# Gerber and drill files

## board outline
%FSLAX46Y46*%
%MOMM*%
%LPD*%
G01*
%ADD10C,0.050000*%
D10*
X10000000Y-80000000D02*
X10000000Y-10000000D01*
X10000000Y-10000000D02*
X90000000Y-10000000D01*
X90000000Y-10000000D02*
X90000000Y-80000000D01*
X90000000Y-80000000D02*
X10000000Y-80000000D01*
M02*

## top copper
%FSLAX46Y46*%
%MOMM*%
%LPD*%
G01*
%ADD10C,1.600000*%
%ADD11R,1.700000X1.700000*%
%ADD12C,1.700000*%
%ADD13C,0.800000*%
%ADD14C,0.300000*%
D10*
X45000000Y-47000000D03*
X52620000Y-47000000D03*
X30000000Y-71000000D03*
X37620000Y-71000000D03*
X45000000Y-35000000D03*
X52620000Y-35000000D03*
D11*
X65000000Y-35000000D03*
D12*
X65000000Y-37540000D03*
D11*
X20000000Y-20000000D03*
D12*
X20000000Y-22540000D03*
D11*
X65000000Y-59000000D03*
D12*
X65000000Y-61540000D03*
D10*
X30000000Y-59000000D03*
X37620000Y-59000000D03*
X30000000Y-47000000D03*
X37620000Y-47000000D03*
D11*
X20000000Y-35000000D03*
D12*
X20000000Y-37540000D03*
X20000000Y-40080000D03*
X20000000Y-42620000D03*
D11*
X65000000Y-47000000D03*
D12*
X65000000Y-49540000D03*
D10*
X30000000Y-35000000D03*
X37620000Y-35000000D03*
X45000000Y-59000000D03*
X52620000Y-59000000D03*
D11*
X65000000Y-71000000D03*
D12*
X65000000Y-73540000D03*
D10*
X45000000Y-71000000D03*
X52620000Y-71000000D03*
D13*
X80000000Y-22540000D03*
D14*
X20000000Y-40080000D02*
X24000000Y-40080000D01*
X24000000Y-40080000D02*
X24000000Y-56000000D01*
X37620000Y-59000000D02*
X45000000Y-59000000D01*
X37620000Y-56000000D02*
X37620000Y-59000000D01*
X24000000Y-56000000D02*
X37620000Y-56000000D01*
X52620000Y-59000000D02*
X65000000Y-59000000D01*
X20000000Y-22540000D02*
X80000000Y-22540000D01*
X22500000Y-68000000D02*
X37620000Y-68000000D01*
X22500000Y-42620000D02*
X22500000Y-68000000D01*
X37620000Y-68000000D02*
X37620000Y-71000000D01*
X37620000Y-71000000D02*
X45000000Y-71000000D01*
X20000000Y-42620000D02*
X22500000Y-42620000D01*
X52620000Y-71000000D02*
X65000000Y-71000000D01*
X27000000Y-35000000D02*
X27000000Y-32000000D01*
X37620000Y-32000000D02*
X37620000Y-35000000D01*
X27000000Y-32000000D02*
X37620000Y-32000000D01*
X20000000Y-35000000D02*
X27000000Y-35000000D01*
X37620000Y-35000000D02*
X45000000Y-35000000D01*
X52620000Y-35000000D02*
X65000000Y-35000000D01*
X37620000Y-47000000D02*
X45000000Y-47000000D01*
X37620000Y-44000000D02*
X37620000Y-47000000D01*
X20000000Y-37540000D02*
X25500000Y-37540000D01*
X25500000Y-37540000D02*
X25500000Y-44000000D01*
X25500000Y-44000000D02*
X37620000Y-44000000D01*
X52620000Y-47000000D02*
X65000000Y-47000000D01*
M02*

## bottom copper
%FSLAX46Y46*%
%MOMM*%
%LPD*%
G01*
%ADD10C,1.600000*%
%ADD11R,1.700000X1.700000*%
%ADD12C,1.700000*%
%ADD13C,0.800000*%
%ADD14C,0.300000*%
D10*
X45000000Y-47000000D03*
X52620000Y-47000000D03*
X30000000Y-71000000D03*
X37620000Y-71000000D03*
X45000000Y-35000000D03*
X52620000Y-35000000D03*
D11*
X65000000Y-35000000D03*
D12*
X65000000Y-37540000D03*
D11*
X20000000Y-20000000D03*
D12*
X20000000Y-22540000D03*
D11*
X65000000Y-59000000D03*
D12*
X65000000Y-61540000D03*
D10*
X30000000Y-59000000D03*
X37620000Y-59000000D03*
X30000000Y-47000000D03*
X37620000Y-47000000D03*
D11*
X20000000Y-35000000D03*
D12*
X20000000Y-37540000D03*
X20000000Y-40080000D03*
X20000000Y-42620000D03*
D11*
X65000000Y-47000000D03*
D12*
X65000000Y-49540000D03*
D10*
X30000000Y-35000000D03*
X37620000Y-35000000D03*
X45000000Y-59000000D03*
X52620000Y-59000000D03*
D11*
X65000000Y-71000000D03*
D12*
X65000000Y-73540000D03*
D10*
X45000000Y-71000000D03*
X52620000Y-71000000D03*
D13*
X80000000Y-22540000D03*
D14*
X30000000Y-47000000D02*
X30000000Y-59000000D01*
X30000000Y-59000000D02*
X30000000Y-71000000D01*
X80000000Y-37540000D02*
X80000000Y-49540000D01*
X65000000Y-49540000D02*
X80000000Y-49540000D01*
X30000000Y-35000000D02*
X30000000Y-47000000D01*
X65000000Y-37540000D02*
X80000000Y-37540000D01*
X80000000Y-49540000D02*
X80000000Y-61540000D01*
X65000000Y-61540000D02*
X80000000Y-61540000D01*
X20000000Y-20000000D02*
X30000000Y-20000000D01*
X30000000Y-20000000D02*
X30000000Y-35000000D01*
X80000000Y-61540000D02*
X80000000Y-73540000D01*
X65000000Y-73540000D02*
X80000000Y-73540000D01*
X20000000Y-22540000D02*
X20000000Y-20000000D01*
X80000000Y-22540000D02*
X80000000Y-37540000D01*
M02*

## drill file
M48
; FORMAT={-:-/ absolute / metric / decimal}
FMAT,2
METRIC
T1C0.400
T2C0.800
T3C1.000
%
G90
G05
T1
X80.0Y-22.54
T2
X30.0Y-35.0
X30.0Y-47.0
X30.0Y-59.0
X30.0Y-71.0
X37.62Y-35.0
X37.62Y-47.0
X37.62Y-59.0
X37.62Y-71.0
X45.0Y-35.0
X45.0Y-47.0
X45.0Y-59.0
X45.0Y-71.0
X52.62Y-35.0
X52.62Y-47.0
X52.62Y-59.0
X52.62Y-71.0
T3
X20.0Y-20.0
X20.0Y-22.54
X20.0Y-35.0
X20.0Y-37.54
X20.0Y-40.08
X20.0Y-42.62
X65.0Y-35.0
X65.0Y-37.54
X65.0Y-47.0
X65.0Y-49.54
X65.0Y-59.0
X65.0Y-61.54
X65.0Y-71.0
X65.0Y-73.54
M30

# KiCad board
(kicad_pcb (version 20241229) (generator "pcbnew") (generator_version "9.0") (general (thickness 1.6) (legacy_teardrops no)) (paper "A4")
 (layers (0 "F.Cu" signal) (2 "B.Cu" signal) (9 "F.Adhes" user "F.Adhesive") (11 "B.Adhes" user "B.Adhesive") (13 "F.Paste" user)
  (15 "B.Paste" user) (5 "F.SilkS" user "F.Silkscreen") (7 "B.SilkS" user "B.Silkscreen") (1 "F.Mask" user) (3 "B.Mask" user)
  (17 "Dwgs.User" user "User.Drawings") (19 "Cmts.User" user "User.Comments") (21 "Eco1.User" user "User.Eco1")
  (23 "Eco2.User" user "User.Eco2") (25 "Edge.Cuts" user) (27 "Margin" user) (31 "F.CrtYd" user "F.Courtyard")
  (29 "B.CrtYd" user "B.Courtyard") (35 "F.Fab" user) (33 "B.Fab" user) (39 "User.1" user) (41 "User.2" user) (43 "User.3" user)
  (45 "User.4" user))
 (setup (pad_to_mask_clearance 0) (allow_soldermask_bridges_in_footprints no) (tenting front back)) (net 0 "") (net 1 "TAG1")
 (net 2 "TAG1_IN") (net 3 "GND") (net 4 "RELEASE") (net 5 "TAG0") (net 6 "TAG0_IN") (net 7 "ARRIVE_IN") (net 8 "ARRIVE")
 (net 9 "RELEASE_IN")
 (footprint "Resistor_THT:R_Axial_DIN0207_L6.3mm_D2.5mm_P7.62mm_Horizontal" (layer "F.Cu") (at 45 47)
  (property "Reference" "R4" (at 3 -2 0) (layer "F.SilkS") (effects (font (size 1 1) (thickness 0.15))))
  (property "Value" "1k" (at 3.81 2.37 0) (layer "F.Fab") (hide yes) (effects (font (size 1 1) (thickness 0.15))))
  (pad "1" thru_hole circle (at 0 0) (size 1.6 1.6) (drill 0.8) (layers "*.Cu" "*.Mask") (remove_unused_layers no) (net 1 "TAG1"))
  (pad "2" thru_hole circle (at 7.62 0) (size 1.6 1.6) (drill 0.8) (layers "*.Cu" "*.Mask") (remove_unused_layers no) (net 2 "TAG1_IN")))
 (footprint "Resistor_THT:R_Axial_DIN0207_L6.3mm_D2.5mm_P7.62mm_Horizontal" (layer "F.Cu") (at 30 71)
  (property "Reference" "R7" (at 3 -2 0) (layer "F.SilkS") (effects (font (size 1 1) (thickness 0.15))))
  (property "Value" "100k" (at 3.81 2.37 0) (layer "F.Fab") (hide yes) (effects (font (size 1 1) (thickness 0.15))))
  (pad "1" thru_hole circle (at 0 0) (size 1.6 1.6) (drill 0.8) (layers "*.Cu" "*.Mask") (remove_unused_layers no) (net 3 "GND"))
  (pad "2" thru_hole circle (at 7.62 0) (size 1.6 1.6) (drill 0.8) (layers "*.Cu" "*.Mask") (remove_unused_layers no) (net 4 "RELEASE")))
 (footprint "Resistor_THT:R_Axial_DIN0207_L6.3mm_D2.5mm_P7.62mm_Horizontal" (layer "F.Cu") (at 45 35)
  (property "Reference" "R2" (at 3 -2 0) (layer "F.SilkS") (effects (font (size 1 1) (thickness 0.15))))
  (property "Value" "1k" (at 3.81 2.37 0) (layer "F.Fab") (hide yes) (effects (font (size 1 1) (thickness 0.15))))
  (pad "1" thru_hole circle (at 0 0) (size 1.6 1.6) (drill 0.8) (layers "*.Cu" "*.Mask") (remove_unused_layers no) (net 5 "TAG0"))
  (pad "2" thru_hole circle (at 7.62 0) (size 1.6 1.6) (drill 0.8) (layers "*.Cu" "*.Mask") (remove_unused_layers no) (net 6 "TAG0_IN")))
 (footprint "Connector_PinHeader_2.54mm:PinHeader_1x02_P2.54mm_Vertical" (layer "F.Cu") (at 65 35)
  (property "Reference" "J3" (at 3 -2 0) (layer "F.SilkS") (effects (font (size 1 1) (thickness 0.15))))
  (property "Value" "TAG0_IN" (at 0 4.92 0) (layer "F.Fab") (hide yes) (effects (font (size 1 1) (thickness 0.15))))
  (pad "1" thru_hole rect (at 0 0) (size 1.7 1.7) (drill 1) (layers "*.Cu" "*.Mask") (remove_unused_layers no) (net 6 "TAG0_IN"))
  (pad "2" thru_hole circle (at 0 2.54) (size 1.7 1.7) (drill 1) (layers "*.Cu" "*.Mask") (remove_unused_layers no) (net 3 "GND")))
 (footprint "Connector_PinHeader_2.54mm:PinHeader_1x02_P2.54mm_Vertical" (layer "F.Cu") (at 20 20)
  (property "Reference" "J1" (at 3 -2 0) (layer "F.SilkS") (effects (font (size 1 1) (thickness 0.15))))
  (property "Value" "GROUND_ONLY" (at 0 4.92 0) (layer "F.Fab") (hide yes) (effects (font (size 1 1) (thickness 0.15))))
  (pad "1" thru_hole rect (at 0 0) (size 1.7 1.7) (drill 1) (layers "*.Cu" "*.Mask") (remove_unused_layers no) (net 3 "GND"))
  (pad "2" thru_hole circle (at 0 2.54) (size 1.7 1.7) (drill 1) (layers "*.Cu" "*.Mask") (remove_unused_layers no) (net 3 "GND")))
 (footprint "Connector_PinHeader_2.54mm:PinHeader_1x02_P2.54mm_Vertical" (layer "F.Cu") (at 65 59)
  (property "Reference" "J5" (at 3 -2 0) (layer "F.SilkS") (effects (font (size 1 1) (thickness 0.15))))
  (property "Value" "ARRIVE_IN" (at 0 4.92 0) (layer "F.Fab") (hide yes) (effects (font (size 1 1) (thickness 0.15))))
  (pad "1" thru_hole rect (at 0 0) (size 1.7 1.7) (drill 1) (layers "*.Cu" "*.Mask") (remove_unused_layers no) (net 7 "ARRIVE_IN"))
  (pad "2" thru_hole circle (at 0 2.54) (size 1.7 1.7) (drill 1) (layers "*.Cu" "*.Mask") (remove_unused_layers no) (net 3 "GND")))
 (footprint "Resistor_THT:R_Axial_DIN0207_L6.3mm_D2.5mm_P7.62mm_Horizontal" (layer "F.Cu") (at 30 59)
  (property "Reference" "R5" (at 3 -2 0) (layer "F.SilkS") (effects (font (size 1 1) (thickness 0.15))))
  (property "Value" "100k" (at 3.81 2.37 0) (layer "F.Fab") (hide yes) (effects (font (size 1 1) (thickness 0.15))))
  (pad "1" thru_hole circle (at 0 0) (size 1.6 1.6) (drill 0.8) (layers "*.Cu" "*.Mask") (remove_unused_layers no) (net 3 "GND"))
  (pad "2" thru_hole circle (at 7.62 0) (size 1.6 1.6) (drill 0.8) (layers "*.Cu" "*.Mask") (remove_unused_layers no) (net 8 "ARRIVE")))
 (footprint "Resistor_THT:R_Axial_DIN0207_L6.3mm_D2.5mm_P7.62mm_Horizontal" (layer "F.Cu") (at 30 47)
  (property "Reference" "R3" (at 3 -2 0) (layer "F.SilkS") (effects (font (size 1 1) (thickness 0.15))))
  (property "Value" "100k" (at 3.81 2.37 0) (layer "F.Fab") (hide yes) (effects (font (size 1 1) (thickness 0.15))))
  (pad "1" thru_hole circle (at 0 0) (size 1.6 1.6) (drill 0.8) (layers "*.Cu" "*.Mask") (remove_unused_layers no) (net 3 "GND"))
  (pad "2" thru_hole circle (at 7.62 0) (size 1.6 1.6) (drill 0.8) (layers "*.Cu" "*.Mask") (remove_unused_layers no) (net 1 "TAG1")))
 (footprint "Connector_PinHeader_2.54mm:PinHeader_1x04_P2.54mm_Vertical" (layer "F.Cu") (at 20 35)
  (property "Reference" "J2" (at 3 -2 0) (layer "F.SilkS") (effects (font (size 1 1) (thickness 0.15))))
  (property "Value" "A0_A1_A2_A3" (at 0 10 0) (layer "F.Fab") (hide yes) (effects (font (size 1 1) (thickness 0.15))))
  (pad "1" thru_hole rect (at 0 0) (size 1.7 1.7) (drill 1) (layers "*.Cu" "*.Mask") (remove_unused_layers no) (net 5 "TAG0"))
  (pad "2" thru_hole circle (at 0 2.54) (size 1.7 1.7) (drill 1) (layers "*.Cu" "*.Mask") (remove_unused_layers no) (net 1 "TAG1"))
  (pad "3" thru_hole circle (at 0 5.08) (size 1.7 1.7) (drill 1) (layers "*.Cu" "*.Mask") (remove_unused_layers no) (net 8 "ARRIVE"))
  (pad "4" thru_hole circle (at 0 7.62) (size 1.7 1.7) (drill 1) (layers "*.Cu" "*.Mask") (remove_unused_layers no) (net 4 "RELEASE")))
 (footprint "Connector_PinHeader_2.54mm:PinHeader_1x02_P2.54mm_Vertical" (layer "F.Cu") (at 65 47)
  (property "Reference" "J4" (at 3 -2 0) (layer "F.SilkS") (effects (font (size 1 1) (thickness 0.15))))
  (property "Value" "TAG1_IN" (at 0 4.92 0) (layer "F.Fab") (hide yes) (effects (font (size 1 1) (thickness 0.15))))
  (pad "1" thru_hole rect (at 0 0) (size 1.7 1.7) (drill 1) (layers "*.Cu" "*.Mask") (remove_unused_layers no) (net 2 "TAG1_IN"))
  (pad "2" thru_hole circle (at 0 2.54) (size 1.7 1.7) (drill 1) (layers "*.Cu" "*.Mask") (remove_unused_layers no) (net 3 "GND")))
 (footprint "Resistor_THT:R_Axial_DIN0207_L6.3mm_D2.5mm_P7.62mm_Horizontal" (layer "F.Cu") (at 30 35)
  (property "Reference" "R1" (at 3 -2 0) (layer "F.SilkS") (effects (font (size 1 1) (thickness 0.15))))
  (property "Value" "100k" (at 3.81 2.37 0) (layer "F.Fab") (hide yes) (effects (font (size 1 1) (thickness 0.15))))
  (pad "1" thru_hole circle (at 0 0) (size 1.6 1.6) (drill 0.8) (layers "*.Cu" "*.Mask") (remove_unused_layers no) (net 3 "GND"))
  (pad "2" thru_hole circle (at 7.62 0) (size 1.6 1.6) (drill 0.8) (layers "*.Cu" "*.Mask") (remove_unused_layers no) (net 5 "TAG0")))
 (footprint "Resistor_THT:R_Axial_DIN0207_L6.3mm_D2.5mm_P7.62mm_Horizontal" (layer "F.Cu") (at 45 59)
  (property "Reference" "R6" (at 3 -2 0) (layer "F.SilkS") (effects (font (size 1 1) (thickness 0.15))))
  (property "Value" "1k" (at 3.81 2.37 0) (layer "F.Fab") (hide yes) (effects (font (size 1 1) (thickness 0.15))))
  (pad "1" thru_hole circle (at 0 0) (size 1.6 1.6) (drill 0.8) (layers "*.Cu" "*.Mask") (remove_unused_layers no) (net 8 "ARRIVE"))
  (pad "2" thru_hole circle (at 7.62 0) (size 1.6 1.6) (drill 0.8) (layers "*.Cu" "*.Mask") (remove_unused_layers no) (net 7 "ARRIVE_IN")))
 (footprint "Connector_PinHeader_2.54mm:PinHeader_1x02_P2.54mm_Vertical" (layer "F.Cu") (at 65 71)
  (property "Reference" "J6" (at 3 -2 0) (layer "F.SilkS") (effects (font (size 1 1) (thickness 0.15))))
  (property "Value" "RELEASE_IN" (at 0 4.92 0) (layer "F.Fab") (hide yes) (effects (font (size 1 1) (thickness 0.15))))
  (pad "1" thru_hole rect (at 0 0) (size 1.7 1.7) (drill 1) (layers "*.Cu" "*.Mask") (remove_unused_layers no) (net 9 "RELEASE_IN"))
  (pad "2" thru_hole circle (at 0 2.54) (size 1.7 1.7) (drill 1) (layers "*.Cu" "*.Mask") (remove_unused_layers no) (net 3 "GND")))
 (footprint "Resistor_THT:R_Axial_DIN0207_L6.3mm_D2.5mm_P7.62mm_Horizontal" (layer "F.Cu") (at 45 71)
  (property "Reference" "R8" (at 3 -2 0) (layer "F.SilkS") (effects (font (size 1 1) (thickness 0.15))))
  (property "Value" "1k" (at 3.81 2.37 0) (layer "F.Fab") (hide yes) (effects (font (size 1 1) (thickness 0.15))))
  (pad "1" thru_hole circle (at 0 0) (size 1.6 1.6) (drill 0.8) (layers "*.Cu" "*.Mask") (remove_unused_layers no) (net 4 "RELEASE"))
  (pad "2" thru_hole circle (at 7.62 0) (size 1.6 1.6) (drill 0.8) (layers "*.Cu" "*.Mask") (remove_unused_layers no) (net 9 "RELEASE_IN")))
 (gr_line (start 10 80) (end 10 10) (stroke (width 0.05) (type default)) (layer "Edge.Cuts"))
 (gr_line (start 10 10) (end 90 10) (stroke (width 0.05) (type default)) (layer "Edge.Cuts"))
 (gr_line (start 90 10) (end 90 80) (stroke (width 0.05) (type default)) (layer "Edge.Cuts"))
 (gr_line (start 90 80) (end 10 80) (stroke (width 0.05) (type default)) (layer "Edge.Cuts"))
 (segment (start 20 40.08) (end 24 40.08) (width 0.3) (layer "F.Cu") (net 8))
 (segment (start 24 40.08) (end 24 56) (width 0.3) (layer "F.Cu") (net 8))
 (segment (start 37.62 59) (end 45 59) (width 0.3) (layer "F.Cu") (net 8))
 (segment (start 37.62 56) (end 37.62 59) (width 0.3) (layer "F.Cu") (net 8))
 (segment (start 24 56) (end 37.62 56) (width 0.3) (layer "F.Cu") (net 8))
 (segment (start 52.62 59) (end 65 59) (width 0.3) (layer "F.Cu") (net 7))
 (segment (start 20 22.54) (end 80 22.54) (width 0.3) (layer "F.Cu") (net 3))
 (via (at 80 22.54) (size 0.8) (drill 0.4) (layers "F.Cu" "B.Cu") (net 3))
 (segment (start 30 47) (end 30 59) (width 0.3) (layer "B.Cu") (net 3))
 (segment (start 30 59) (end 30 71) (width 0.3) (layer "B.Cu") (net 3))
 (segment (start 80 37.54) (end 80 49.54) (width 0.3) (layer "B.Cu") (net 3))
 (segment (start 65 49.54) (end 80 49.54) (width 0.3) (layer "B.Cu") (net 3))
 (segment (start 30 35) (end 30 47) (width 0.3) (layer "B.Cu") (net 3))
 (segment (start 65 37.54) (end 80 37.54) (width 0.3) (layer "B.Cu") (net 3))
 (segment (start 80 49.54) (end 80 61.54) (width 0.3) (layer "B.Cu") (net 3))
 (segment (start 65 61.54) (end 80 61.54) (width 0.3) (layer "B.Cu") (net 3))
 (segment (start 20 20) (end 30 20) (width 0.3) (layer "B.Cu") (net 3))
 (segment (start 30 20) (end 30 35) (width 0.3) (layer "B.Cu") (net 3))
 (segment (start 80 61.54) (end 80 73.54) (width 0.3) (layer "B.Cu") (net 3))
 (segment (start 65 73.54) (end 80 73.54) (width 0.3) (layer "B.Cu") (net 3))
 (segment (start 20 22.54) (end 20 20) (width 0.3) (layer "B.Cu") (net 3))
 (segment (start 80 22.54) (end 80 37.54) (width 0.3) (layer "B.Cu") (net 3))
 (segment (start 22.5 68) (end 37.62 68) (width 0.3) (layer "F.Cu") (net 4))
 (segment (start 22.5 42.62) (end 22.5 68) (width 0.3) (layer "F.Cu") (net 4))
 (segment (start 37.62 68) (end 37.62 71) (width 0.3) (layer "F.Cu") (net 4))
 (segment (start 37.62 71) (end 45 71) (width 0.3) (layer "F.Cu") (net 4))
 (segment (start 20 42.62) (end 22.5 42.62) (width 0.3) (layer "F.Cu") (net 4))
 (segment (start 52.62 71) (end 65 71) (width 0.3) (layer "F.Cu") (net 9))
 (segment (start 27 35) (end 27 32) (width 0.3) (layer "F.Cu") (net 5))
 (segment (start 37.62 32) (end 37.62 35) (width 0.3) (layer "F.Cu") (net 5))
 (segment (start 27 32) (end 37.62 32) (width 0.3) (layer "F.Cu") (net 5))
 (segment (start 20 35) (end 27 35) (width 0.3) (layer "F.Cu") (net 5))
 (segment (start 37.62 35) (end 45 35) (width 0.3) (layer "F.Cu") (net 5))
 (segment (start 52.62 35) (end 65 35) (width 0.3) (layer "F.Cu") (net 6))
 (segment (start 37.62 47) (end 45 47) (width 0.3) (layer "F.Cu") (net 1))
 (segment (start 37.62 44) (end 37.62 47) (width 0.3) (layer "F.Cu") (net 1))
 (segment (start 20 37.54) (end 25.5 37.54) (width 0.3) (layer "F.Cu") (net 1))
 (segment (start 25.5 37.54) (end 25.5 44) (width 0.3) (layer "F.Cu") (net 1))
 (segment (start 25.5 44) (end 37.62 44) (width 0.3) (layer "F.Cu") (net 1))
 (segment (start 52.62 47) (end 65 47) (width 0.3) (layer "F.Cu") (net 2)))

